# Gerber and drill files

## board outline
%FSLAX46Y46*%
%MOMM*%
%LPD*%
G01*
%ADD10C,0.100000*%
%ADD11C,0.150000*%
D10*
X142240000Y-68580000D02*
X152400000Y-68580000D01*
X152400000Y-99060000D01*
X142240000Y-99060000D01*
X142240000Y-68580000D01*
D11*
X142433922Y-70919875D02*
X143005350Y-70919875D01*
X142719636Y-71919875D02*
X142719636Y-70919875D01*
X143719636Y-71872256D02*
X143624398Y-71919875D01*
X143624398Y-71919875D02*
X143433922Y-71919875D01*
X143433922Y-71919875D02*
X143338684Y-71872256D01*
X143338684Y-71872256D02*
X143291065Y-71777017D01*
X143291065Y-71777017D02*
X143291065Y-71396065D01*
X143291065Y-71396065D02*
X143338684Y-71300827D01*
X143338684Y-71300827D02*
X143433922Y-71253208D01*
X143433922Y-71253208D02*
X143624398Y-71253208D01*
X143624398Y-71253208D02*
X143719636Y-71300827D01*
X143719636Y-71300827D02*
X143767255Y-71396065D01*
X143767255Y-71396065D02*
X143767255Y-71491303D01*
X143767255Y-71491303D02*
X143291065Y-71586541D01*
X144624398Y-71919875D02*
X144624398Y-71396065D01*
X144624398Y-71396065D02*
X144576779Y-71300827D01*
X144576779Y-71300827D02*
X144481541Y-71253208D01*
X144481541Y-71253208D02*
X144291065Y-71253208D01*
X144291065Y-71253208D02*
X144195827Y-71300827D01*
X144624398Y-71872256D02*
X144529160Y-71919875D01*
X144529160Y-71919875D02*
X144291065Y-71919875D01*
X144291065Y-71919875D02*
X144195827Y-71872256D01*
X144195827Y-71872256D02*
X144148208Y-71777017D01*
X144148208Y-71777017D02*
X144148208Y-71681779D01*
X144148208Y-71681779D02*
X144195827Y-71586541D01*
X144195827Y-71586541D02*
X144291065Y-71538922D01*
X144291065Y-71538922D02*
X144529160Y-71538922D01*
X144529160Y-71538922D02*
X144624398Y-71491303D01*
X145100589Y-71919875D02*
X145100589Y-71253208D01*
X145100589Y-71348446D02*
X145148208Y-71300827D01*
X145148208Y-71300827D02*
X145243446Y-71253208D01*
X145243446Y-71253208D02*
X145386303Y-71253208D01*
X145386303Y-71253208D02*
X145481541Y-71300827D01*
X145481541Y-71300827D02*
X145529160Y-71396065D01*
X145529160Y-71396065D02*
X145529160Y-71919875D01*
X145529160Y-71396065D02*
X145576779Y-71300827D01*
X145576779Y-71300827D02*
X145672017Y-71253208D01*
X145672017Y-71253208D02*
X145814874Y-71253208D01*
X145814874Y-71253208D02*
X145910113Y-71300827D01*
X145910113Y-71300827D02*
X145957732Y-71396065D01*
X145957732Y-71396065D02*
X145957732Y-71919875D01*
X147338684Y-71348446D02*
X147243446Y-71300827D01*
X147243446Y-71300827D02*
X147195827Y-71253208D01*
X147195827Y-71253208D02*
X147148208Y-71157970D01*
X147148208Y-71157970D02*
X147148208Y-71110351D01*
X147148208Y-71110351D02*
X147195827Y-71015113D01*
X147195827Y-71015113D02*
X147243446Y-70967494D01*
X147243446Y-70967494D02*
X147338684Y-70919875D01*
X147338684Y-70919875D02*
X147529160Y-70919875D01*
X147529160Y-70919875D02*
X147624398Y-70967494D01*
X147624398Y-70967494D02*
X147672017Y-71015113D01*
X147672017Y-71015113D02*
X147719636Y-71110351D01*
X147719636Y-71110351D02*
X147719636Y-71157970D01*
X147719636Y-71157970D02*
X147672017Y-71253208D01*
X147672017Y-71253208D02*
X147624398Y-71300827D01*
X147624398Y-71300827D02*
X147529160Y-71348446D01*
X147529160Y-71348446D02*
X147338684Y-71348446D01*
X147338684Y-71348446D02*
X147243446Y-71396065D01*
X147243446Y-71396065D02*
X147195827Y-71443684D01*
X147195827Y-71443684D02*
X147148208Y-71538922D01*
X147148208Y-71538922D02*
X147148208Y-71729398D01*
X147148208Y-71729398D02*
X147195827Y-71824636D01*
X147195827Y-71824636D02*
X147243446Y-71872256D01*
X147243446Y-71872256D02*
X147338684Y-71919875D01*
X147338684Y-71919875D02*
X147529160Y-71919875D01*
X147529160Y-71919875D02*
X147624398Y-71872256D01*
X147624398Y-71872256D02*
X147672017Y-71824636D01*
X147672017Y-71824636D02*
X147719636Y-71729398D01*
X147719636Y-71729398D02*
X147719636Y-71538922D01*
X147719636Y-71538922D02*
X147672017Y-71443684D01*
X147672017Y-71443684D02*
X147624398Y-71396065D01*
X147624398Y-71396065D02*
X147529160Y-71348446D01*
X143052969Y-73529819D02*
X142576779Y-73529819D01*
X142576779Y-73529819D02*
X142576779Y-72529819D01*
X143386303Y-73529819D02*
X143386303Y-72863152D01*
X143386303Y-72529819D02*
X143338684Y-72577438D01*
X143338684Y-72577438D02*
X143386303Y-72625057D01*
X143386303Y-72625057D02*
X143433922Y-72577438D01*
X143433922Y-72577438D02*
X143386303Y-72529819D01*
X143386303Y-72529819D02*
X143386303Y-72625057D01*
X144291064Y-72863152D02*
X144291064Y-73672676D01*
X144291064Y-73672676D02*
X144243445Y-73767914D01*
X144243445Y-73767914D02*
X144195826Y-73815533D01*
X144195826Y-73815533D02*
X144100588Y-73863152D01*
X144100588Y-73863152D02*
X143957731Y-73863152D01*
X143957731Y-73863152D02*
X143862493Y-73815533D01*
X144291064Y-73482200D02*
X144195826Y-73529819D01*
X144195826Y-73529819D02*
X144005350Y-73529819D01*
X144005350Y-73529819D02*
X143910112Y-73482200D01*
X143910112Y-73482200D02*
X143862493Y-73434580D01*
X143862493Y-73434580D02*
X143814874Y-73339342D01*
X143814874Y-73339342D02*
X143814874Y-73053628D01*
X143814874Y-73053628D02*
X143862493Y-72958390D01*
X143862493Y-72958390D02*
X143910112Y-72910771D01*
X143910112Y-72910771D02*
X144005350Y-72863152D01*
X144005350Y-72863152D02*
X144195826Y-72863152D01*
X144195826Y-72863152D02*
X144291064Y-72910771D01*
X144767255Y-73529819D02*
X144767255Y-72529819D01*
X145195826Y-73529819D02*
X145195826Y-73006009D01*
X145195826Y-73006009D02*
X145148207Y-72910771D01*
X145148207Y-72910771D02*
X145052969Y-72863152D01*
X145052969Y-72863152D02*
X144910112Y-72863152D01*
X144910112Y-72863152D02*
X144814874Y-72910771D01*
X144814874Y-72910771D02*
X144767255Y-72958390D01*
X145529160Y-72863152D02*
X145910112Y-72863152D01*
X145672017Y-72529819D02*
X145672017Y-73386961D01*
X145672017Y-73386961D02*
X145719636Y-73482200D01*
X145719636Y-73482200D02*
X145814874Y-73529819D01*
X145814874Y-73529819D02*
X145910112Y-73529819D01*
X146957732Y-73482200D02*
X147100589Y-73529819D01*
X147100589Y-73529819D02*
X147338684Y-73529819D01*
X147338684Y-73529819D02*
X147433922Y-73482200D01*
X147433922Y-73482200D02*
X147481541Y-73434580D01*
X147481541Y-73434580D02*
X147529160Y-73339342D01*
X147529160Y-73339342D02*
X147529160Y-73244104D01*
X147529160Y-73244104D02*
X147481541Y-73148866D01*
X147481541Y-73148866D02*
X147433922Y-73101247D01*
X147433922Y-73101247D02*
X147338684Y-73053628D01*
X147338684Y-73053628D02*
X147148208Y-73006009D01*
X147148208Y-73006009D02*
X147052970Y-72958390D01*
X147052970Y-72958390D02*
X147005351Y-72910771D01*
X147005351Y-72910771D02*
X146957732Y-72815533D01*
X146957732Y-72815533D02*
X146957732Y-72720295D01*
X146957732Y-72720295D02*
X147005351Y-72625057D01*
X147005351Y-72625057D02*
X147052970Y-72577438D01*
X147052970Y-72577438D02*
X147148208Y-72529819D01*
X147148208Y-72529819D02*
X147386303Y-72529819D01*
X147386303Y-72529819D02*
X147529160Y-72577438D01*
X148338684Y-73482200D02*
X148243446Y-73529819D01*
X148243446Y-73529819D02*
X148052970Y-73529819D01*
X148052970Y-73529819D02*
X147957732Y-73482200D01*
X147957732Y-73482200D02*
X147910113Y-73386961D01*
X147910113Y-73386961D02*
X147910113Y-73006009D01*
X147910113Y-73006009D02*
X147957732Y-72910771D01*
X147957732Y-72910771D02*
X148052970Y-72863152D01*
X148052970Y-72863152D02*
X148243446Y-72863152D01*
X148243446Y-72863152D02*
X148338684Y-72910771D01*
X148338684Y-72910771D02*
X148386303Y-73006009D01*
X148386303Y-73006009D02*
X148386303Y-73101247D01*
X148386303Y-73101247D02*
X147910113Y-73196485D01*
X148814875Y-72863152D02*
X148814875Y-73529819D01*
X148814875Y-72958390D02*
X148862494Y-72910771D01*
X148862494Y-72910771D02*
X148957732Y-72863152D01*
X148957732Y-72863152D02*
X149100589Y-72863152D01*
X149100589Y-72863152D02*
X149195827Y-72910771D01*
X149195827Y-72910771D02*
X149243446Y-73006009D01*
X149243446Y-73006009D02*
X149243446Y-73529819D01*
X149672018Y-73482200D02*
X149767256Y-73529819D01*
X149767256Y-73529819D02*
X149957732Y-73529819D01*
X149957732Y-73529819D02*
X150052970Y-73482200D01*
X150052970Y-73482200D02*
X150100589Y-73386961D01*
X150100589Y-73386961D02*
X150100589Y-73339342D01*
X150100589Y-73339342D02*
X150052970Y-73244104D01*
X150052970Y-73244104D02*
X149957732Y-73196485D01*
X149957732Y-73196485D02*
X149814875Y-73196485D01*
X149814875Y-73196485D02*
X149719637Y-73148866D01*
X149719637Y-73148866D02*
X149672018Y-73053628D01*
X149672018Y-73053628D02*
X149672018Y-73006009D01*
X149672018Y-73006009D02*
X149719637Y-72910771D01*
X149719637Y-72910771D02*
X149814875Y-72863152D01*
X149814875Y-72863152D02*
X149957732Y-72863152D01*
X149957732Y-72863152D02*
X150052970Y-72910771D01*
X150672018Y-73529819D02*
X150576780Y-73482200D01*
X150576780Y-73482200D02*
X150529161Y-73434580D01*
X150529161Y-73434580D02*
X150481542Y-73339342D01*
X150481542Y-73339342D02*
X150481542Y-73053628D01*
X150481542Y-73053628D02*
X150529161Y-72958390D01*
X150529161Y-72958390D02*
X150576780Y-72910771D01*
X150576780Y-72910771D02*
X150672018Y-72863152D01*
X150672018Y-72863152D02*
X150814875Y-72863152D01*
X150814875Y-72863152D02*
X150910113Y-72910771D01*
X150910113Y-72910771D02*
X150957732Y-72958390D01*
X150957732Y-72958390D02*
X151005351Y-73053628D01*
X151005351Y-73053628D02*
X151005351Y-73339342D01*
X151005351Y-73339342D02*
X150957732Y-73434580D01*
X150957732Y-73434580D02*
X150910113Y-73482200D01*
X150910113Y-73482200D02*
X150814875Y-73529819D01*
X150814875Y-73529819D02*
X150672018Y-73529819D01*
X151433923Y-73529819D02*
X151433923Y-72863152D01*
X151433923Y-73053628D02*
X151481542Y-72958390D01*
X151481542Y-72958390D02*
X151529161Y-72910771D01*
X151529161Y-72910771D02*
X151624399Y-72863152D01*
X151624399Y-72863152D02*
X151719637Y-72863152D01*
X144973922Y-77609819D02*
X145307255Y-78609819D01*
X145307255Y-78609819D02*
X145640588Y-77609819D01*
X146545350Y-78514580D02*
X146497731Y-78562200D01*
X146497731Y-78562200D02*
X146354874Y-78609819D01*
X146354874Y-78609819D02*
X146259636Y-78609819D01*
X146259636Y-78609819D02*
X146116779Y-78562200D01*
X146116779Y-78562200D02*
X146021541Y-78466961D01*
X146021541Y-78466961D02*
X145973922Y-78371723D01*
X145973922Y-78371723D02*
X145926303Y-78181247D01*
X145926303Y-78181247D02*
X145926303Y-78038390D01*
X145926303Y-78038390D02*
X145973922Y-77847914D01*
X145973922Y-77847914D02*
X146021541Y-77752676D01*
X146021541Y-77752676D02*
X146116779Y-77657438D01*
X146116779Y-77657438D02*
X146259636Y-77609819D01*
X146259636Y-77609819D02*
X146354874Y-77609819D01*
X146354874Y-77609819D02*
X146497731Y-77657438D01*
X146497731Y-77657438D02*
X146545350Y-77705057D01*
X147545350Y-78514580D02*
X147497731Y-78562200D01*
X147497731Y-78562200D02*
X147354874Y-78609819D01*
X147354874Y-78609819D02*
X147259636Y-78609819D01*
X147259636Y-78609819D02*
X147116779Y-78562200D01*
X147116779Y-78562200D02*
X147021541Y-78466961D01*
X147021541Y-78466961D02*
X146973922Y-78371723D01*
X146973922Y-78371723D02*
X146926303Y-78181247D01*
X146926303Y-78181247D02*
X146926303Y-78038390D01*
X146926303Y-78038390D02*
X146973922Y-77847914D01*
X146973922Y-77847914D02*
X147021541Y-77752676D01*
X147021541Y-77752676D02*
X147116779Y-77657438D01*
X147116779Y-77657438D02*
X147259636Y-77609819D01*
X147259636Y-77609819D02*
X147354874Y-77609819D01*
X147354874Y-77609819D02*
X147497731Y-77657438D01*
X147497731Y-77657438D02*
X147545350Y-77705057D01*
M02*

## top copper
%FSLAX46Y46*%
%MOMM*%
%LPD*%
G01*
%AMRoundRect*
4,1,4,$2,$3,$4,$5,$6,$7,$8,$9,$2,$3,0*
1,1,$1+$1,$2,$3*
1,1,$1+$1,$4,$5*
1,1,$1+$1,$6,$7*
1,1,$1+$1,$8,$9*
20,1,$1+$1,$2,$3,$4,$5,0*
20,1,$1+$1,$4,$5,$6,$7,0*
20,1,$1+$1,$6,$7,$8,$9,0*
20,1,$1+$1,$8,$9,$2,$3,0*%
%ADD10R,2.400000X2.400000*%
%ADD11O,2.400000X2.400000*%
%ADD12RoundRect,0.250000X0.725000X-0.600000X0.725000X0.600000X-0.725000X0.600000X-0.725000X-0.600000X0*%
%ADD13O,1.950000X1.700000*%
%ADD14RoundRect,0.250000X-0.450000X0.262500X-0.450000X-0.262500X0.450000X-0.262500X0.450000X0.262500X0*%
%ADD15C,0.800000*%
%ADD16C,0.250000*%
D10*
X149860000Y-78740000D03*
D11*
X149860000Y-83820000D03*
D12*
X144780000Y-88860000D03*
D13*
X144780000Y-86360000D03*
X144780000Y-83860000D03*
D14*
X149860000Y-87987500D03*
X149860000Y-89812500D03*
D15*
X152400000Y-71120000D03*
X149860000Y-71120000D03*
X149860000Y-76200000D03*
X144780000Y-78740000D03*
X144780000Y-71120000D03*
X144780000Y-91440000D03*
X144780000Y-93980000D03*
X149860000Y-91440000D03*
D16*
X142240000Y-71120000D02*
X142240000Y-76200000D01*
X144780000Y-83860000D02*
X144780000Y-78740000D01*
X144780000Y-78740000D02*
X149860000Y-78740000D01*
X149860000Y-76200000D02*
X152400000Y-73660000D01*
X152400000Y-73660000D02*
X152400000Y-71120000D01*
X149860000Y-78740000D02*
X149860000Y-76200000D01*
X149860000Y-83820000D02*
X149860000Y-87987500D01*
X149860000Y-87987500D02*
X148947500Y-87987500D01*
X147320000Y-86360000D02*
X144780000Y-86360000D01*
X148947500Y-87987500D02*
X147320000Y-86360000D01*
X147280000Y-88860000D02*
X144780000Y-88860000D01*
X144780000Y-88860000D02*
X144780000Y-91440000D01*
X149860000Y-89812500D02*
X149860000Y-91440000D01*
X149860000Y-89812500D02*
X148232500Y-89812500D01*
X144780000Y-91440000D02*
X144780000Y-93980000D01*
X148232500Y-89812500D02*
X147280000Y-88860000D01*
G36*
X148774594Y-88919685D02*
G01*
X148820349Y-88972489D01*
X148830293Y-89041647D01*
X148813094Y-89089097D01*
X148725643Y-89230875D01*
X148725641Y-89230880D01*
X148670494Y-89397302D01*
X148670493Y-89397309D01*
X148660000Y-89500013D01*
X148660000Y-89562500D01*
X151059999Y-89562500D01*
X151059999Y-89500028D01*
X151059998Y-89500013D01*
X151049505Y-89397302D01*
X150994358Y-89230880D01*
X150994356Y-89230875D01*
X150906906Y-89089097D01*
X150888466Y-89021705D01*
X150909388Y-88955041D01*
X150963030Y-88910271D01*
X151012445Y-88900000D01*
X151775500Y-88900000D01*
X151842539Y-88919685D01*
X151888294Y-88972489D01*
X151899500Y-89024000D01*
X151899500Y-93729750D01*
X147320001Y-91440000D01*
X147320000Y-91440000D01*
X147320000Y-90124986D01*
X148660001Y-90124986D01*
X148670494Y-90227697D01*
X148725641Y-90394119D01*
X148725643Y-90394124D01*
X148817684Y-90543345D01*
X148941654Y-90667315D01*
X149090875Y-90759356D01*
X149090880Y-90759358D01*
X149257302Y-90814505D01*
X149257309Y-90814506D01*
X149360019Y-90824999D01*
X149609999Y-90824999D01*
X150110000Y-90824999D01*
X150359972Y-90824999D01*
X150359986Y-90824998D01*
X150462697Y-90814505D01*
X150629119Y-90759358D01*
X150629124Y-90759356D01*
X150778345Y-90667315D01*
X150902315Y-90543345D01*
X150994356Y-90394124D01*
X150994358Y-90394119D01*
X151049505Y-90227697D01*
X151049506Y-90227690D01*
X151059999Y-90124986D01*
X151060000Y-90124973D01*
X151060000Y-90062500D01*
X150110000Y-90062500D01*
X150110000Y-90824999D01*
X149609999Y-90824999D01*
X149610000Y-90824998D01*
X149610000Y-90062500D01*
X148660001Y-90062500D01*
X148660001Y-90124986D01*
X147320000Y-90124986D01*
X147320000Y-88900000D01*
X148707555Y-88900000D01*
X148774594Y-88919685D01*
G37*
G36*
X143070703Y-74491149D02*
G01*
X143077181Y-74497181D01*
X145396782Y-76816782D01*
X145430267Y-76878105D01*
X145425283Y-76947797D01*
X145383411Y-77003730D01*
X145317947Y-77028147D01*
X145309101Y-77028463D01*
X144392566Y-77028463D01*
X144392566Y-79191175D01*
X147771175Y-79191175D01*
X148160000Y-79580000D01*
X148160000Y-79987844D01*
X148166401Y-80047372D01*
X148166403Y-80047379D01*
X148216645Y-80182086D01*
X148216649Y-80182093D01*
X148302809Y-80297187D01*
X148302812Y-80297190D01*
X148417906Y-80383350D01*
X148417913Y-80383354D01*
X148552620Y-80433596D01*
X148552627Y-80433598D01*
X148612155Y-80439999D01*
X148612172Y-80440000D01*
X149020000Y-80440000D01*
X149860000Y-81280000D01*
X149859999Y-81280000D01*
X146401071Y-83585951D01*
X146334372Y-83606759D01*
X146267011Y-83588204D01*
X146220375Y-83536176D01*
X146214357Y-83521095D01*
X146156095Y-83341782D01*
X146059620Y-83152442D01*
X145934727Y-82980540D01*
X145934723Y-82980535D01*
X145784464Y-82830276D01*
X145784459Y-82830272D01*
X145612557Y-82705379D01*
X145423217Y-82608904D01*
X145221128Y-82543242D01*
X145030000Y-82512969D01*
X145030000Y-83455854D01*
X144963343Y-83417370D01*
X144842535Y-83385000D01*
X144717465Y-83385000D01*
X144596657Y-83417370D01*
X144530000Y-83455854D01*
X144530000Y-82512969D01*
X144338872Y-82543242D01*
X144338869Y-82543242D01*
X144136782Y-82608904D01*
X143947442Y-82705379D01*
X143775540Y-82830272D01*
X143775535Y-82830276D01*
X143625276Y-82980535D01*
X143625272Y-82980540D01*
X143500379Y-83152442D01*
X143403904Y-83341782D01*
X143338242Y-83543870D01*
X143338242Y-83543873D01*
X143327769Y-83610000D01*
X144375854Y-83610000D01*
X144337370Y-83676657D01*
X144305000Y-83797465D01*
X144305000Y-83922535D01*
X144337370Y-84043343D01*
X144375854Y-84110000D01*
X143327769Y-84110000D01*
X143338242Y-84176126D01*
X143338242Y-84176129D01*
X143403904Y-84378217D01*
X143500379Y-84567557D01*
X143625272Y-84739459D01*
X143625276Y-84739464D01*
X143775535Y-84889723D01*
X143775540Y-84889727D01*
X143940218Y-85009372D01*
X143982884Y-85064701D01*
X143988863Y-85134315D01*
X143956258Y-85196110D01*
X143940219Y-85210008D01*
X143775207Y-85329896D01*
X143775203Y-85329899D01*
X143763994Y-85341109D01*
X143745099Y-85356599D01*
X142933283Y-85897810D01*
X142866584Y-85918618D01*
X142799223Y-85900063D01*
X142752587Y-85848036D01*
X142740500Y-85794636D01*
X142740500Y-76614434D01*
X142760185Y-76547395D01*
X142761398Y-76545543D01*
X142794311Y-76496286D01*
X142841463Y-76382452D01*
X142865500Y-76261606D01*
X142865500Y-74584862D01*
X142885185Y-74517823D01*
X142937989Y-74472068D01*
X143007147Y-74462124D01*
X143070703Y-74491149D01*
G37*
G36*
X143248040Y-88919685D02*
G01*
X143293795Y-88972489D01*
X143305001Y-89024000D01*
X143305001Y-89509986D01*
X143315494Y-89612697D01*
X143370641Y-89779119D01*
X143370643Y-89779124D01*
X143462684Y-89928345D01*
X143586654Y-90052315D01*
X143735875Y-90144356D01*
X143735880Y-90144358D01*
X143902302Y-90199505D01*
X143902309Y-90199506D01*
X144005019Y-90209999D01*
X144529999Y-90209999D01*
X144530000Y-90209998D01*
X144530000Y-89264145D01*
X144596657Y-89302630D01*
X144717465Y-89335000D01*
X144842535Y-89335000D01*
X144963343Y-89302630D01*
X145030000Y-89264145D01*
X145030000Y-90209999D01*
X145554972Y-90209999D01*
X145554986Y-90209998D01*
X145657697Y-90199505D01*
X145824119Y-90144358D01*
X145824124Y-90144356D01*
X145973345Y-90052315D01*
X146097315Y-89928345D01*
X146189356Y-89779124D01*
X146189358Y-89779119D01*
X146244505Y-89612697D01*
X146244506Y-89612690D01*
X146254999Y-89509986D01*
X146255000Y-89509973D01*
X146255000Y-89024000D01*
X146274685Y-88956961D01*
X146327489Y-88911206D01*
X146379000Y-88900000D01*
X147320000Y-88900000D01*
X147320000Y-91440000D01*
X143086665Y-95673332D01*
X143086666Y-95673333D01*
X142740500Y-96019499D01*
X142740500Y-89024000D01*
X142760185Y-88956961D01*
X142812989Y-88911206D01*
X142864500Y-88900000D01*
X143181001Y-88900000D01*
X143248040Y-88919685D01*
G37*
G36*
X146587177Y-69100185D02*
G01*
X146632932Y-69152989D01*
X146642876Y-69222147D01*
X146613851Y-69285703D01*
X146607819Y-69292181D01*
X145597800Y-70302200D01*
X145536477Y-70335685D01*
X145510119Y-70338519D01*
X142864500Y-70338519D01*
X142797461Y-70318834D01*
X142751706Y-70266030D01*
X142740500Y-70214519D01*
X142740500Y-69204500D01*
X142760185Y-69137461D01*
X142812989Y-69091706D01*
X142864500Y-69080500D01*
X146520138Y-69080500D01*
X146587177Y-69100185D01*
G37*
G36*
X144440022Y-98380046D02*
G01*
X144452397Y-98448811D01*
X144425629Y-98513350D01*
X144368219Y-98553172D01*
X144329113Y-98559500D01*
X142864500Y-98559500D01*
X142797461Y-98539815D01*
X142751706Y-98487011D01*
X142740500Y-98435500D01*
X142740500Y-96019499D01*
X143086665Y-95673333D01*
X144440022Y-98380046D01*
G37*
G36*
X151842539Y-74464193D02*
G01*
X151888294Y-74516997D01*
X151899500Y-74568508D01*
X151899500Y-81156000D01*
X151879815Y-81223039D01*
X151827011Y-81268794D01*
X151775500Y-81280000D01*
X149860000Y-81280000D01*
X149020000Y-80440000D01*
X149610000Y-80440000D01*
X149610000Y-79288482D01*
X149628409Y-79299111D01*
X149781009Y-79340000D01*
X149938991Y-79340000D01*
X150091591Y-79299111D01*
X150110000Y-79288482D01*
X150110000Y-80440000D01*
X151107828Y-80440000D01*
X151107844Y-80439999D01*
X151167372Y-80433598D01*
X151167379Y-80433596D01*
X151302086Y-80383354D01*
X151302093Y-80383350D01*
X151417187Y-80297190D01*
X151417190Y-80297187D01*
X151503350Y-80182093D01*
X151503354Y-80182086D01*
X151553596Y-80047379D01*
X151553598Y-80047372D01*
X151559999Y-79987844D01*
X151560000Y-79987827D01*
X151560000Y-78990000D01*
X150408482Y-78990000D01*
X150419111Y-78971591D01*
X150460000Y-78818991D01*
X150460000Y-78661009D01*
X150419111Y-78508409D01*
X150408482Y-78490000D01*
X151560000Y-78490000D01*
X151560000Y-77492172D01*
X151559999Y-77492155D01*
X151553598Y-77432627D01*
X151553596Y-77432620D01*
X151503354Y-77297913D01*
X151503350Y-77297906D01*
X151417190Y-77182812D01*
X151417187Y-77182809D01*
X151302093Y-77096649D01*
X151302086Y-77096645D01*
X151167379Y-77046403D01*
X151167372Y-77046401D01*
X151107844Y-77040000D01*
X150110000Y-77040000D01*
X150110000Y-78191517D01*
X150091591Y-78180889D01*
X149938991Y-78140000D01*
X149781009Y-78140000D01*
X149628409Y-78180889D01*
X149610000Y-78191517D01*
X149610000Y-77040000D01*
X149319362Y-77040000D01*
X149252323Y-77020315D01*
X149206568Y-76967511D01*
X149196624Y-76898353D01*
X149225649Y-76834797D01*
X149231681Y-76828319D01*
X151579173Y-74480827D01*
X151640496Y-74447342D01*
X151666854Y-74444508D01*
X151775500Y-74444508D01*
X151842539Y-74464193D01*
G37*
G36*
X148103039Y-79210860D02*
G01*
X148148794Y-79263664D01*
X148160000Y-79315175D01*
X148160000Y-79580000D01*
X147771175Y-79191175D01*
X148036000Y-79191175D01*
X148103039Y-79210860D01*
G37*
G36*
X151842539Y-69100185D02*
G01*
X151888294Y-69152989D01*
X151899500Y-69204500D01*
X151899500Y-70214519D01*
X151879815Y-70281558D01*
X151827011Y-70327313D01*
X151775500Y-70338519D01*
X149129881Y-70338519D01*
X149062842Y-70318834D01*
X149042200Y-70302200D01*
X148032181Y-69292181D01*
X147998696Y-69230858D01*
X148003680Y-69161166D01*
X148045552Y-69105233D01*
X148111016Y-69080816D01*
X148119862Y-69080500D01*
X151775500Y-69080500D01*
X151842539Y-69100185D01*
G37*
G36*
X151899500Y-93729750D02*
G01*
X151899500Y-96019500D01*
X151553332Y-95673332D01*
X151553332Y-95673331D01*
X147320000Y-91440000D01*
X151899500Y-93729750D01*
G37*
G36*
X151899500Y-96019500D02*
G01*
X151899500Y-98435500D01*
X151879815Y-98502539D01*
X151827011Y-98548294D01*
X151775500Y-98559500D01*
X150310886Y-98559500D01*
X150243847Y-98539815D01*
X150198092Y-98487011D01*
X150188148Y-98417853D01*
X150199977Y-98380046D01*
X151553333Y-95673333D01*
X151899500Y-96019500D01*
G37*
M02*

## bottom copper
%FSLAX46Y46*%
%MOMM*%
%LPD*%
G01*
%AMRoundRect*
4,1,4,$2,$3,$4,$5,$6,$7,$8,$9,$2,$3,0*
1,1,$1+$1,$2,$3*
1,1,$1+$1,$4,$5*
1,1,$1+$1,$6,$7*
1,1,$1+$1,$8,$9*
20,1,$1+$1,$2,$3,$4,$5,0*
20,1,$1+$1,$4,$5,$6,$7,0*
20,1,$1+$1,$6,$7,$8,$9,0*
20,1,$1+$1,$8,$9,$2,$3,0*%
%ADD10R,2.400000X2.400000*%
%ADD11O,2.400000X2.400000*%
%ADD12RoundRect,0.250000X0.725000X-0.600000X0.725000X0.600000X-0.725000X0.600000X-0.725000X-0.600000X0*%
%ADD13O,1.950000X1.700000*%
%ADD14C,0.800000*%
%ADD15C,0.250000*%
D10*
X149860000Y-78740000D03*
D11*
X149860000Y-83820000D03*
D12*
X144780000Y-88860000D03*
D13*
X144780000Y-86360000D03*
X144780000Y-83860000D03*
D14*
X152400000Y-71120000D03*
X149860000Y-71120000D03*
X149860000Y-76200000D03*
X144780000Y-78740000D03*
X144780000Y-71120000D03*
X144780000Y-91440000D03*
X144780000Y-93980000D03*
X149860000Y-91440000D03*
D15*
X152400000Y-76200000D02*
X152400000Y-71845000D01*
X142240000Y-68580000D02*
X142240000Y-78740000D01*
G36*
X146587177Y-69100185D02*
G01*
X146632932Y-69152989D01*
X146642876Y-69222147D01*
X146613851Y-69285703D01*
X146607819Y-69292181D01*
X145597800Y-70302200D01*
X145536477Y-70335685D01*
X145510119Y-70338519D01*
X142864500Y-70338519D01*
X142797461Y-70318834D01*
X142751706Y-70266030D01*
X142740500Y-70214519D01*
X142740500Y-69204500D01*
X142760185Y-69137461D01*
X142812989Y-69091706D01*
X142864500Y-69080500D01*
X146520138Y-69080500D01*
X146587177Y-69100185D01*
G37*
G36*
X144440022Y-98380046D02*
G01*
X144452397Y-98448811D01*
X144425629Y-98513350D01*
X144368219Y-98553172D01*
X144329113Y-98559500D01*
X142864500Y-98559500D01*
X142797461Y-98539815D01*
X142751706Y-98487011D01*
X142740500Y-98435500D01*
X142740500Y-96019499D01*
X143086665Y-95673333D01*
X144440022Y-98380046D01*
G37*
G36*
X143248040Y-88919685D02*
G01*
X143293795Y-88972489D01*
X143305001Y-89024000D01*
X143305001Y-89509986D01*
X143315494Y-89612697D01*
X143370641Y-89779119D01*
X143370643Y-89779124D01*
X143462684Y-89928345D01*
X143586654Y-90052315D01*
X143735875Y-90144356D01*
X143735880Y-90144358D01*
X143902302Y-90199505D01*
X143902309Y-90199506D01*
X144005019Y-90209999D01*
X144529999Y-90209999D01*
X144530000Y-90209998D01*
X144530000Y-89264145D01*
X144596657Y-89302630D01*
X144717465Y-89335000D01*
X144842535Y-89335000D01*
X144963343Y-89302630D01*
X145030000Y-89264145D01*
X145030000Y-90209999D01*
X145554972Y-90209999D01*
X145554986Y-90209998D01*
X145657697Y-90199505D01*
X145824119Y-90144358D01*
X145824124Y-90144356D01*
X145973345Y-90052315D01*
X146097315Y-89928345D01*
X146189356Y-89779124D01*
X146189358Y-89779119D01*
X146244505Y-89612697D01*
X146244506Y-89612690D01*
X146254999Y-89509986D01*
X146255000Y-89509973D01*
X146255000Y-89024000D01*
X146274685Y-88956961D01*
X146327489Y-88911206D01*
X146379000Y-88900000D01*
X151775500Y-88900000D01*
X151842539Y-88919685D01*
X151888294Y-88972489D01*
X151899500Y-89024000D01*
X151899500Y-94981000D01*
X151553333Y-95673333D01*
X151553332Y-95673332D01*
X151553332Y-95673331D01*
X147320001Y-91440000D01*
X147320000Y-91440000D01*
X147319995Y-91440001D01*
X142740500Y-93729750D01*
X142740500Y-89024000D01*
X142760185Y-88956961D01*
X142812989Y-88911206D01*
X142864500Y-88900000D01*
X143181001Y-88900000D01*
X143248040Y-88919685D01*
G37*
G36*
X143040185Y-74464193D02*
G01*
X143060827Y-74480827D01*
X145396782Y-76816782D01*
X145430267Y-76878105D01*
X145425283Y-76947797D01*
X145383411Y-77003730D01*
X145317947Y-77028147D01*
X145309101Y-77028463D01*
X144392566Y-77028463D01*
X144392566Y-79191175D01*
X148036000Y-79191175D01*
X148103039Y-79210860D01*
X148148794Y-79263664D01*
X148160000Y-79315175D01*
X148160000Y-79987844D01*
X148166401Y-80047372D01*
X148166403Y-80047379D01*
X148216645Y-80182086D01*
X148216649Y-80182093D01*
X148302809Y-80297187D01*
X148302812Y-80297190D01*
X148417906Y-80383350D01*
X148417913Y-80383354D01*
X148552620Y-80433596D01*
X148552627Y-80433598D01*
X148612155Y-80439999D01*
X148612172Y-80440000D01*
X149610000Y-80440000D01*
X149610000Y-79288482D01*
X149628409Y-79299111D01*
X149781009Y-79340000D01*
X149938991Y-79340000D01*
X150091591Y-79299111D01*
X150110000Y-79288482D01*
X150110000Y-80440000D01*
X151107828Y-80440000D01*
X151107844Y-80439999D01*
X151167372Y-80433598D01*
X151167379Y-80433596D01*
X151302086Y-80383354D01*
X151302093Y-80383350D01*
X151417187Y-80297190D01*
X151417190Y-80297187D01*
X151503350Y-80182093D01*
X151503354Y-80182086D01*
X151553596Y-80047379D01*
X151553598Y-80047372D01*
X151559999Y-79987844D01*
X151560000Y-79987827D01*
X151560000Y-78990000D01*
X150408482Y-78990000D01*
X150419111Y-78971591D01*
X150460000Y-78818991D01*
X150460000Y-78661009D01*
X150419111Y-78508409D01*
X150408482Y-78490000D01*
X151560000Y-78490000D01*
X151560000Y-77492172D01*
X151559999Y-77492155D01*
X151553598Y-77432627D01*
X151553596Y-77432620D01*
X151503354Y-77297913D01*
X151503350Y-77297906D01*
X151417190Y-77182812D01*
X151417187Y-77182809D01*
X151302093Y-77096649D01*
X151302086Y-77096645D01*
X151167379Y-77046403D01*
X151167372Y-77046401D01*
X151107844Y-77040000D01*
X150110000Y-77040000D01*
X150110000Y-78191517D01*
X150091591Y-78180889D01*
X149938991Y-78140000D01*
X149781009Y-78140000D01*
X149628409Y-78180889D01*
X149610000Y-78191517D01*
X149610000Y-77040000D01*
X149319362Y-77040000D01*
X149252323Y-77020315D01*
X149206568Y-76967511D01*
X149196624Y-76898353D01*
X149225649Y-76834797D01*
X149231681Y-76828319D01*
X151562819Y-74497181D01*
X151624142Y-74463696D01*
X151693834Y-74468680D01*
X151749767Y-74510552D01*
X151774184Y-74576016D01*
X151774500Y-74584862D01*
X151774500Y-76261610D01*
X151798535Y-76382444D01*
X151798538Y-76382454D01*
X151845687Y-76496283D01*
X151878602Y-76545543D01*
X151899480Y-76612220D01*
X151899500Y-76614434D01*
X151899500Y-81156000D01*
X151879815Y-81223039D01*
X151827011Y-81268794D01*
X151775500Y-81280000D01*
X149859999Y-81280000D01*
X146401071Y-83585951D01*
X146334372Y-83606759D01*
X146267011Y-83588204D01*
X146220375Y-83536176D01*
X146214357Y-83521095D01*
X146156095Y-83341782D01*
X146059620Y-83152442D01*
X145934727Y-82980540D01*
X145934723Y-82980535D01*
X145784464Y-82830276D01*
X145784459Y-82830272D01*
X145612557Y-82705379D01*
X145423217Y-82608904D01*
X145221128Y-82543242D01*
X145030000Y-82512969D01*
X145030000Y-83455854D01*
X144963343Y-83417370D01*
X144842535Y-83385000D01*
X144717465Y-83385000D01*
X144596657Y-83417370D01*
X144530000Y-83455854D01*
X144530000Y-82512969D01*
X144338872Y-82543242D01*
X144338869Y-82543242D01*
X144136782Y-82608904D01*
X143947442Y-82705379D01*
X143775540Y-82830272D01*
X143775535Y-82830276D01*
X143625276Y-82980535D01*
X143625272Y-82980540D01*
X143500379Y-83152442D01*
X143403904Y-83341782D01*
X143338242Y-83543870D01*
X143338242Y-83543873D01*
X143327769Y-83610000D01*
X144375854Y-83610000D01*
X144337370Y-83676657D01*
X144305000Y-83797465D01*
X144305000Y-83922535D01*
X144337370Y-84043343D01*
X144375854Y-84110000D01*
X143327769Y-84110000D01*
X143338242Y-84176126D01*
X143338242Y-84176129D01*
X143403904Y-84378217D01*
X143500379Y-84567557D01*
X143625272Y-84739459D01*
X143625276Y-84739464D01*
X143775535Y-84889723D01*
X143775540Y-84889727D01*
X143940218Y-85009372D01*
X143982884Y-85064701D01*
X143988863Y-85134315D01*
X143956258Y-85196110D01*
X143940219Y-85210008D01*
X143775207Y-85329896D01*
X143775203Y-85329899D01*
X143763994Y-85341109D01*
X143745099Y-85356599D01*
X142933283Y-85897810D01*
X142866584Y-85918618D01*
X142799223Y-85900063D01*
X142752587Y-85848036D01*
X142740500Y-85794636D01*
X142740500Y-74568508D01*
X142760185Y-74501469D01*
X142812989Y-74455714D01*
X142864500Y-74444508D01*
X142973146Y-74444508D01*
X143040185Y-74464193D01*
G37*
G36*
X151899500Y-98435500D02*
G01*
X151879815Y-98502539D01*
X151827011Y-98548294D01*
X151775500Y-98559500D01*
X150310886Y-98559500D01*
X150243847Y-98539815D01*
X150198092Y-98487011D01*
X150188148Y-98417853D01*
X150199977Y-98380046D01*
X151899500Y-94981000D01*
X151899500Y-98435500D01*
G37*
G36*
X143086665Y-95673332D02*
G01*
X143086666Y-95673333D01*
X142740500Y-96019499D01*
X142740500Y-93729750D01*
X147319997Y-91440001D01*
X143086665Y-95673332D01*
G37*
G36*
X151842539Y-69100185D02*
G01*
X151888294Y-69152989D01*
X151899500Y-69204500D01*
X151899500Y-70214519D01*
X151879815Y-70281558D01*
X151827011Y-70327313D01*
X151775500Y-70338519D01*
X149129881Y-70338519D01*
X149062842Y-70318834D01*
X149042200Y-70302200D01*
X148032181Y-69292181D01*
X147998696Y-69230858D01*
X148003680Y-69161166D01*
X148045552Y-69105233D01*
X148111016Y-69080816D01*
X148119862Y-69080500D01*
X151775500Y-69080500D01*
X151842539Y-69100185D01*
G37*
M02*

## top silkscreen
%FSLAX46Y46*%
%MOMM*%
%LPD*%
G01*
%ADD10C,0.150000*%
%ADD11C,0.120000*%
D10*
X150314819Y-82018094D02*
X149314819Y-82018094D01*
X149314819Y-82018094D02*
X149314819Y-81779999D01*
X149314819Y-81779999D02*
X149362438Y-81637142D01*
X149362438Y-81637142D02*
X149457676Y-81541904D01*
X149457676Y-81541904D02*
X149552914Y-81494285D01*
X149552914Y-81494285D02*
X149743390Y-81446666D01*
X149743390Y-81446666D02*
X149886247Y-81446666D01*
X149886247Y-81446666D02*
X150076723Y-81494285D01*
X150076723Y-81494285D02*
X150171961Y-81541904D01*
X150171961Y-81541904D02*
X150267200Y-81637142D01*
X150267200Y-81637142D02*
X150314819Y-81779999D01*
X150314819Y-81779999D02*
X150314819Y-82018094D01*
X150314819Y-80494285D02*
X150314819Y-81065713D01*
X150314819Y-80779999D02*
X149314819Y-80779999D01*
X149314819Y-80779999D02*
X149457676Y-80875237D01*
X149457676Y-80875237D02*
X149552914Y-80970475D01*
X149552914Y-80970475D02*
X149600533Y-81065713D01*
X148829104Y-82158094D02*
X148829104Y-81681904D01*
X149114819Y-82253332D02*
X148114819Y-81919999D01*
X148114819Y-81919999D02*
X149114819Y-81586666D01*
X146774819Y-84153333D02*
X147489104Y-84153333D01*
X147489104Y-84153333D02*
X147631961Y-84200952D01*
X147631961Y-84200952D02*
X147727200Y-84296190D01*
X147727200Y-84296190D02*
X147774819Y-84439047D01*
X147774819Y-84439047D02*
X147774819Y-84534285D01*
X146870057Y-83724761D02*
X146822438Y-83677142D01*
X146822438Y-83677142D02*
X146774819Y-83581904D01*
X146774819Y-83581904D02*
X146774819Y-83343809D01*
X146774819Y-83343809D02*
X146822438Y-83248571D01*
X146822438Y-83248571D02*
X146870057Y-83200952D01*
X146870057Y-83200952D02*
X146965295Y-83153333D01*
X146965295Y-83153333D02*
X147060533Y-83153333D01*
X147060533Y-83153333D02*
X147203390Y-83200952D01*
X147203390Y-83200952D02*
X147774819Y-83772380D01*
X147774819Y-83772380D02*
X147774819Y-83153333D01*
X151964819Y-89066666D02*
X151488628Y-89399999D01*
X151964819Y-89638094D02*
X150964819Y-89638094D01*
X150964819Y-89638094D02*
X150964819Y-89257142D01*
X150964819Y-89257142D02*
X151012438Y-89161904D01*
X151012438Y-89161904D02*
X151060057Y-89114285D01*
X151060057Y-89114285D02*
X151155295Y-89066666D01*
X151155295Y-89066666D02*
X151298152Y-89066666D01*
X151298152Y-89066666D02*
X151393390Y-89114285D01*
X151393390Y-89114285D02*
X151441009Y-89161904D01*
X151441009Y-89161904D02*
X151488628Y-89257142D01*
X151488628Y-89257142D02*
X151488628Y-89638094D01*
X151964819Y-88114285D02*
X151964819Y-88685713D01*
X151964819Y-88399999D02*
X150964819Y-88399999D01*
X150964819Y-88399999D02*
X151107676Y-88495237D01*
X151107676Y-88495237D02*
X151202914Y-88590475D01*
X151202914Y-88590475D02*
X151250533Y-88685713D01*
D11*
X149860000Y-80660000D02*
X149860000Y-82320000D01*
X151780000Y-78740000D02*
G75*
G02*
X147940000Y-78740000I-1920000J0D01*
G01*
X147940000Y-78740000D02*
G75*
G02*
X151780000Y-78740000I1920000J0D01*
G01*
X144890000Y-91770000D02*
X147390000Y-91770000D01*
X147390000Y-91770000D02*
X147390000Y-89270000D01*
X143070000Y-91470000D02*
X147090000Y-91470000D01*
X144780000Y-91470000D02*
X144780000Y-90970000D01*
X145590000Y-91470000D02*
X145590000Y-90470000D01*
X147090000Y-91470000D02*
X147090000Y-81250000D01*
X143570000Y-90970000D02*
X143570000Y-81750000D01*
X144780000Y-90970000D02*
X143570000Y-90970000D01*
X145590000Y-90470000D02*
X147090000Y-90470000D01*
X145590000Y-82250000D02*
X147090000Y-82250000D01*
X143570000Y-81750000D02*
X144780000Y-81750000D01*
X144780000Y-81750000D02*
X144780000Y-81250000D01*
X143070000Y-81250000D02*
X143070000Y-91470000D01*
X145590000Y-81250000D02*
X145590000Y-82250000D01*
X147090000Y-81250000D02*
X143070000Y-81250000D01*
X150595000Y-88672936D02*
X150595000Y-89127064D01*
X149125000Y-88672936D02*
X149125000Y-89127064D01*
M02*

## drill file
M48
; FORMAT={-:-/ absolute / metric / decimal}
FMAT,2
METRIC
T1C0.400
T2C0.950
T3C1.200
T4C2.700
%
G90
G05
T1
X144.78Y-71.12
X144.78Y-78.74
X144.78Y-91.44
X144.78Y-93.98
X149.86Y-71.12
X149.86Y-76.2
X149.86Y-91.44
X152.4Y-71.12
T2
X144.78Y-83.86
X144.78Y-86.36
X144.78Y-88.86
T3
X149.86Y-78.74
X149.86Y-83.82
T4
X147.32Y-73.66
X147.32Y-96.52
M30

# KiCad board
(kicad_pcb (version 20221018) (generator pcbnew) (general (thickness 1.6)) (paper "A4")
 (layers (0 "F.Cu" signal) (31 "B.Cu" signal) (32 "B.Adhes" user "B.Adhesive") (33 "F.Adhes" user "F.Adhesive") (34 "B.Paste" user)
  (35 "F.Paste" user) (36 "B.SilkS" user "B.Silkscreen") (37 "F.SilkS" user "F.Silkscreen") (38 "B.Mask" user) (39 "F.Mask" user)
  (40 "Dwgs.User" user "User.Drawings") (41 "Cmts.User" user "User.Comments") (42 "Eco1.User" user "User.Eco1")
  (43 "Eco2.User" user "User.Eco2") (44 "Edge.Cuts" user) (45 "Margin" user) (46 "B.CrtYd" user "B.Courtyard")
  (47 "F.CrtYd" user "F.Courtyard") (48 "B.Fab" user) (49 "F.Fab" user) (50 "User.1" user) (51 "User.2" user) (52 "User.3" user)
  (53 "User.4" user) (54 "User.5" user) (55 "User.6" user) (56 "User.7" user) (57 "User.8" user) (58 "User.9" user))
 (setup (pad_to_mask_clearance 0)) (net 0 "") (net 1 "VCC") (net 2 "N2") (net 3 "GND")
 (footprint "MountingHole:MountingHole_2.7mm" (layer "F.Cu") (at 147.32 96.52)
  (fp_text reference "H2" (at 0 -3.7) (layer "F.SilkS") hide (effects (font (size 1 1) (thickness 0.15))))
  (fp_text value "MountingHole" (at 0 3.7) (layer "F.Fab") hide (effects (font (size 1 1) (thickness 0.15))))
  (pad "" np_thru_hole circle (at 0 0) (size 2.7 2.7) (drill 2.7) (layers "*.Cu" "*.Mask")))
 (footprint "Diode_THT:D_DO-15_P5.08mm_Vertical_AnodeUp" (layer "F.Cu") (at 149.86 78.74 -90)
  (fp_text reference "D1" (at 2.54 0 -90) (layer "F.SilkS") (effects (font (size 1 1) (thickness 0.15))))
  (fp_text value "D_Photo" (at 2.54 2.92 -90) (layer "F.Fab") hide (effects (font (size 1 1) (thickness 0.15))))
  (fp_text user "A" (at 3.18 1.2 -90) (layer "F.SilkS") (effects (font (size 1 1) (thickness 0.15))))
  (fp_line (start 1.92 0) (end 3.58 0) (stroke (width 0.12) (type solid)) (layer "F.SilkS"))
  (fp_circle (center 0 0) (end 1.92 0) (stroke (width 0.12) (type solid)) (fill none) (layer "F.SilkS"))
  (pad "1" thru_hole rect (at 0 0 270) (size 2.4 2.4) (drill 1.2) (layers "*.Cu" "*.Mask") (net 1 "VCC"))
  (pad "2" thru_hole oval (at 5.08 0 270) (size 2.4 2.4) (drill 1.2) (layers "*.Cu" "*.Mask") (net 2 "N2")))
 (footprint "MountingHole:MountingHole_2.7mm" (layer "F.Cu") (at 147.32 73.66)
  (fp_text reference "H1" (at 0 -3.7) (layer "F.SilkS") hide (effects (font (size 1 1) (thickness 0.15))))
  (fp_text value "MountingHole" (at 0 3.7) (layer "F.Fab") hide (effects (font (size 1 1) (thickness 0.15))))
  (pad "" np_thru_hole circle (at 0 0) (size 2.7 2.7) (drill 2.7) (layers "*.Cu" "*.Mask")))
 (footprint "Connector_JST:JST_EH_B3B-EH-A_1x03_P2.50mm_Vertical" (layer "F.Cu") (at 144.78 88.86 90)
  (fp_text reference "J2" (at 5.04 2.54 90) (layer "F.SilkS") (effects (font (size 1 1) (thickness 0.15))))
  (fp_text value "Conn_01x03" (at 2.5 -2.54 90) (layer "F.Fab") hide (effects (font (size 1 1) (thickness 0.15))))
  (fp_line (start -2.91 0.11) (end -2.91 2.61) (stroke (width 0.12) (type solid)) (layer "F.SilkS"))
  (fp_line (start -2.91 2.61) (end -0.41 2.61) (stroke (width 0.12) (type solid)) (layer "F.SilkS"))
  (fp_line (start -2.61 -1.71) (end -2.61 2.31) (stroke (width 0.12) (type solid)) (layer "F.SilkS"))
  (fp_line (start -2.61 0) (end -2.11 0) (stroke (width 0.12) (type solid)) (layer "F.SilkS"))
  (fp_line (start -2.61 0.81) (end -1.61 0.81) (stroke (width 0.12) (type solid)) (layer "F.SilkS"))
  (fp_line (start -2.61 2.31) (end 7.61 2.31) (stroke (width 0.12) (type solid)) (layer "F.SilkS"))
  (fp_line (start -2.11 -1.21) (end 7.11 -1.21) (stroke (width 0.12) (type solid)) (layer "F.SilkS"))
  (fp_line (start -2.11 0) (end -2.11 -1.21) (stroke (width 0.12) (type solid)) (layer "F.SilkS"))
  (fp_line (start -1.61 0.81) (end -1.61 2.31) (stroke (width 0.12) (type solid)) (layer "F.SilkS"))
  (fp_line (start 6.61 0.81) (end 6.61 2.31) (stroke (width 0.12) (type solid)) (layer "F.SilkS"))
  (fp_line (start 7.11 -1.21) (end 7.11 0) (stroke (width 0.12) (type solid)) (layer "F.SilkS"))
  (fp_line (start 7.11 0) (end 7.61 0) (stroke (width 0.12) (type solid)) (layer "F.SilkS"))
  (fp_line (start 7.61 -1.71) (end -2.61 -1.71) (stroke (width 0.12) (type solid)) (layer "F.SilkS"))
  (fp_line (start 7.61 0.81) (end 6.61 0.81) (stroke (width 0.12) (type solid)) (layer "F.SilkS"))
  (fp_line (start 7.61 2.31) (end 7.61 -1.71) (stroke (width 0.12) (type solid)) (layer "F.SilkS"))
  (pad "1" thru_hole roundrect (at 0 0 90) (size 1.7 1.95) (drill 0.95) (layers "*.Cu" "*.Mask") (roundrect_rratio 0.1470588235)
   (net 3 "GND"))
  (pad "2" thru_hole oval (at 2.5 0 90) (size 1.7 1.95) (drill 0.95) (layers "*.Cu" "*.Mask") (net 2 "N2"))
  (pad "3" thru_hole oval (at 5 0 90) (size 1.7 1.95) (drill 0.95) (layers "*.Cu" "*.Mask") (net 1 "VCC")))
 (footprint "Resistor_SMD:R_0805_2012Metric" (layer "F.Cu") (at 149.86 88.9 -90)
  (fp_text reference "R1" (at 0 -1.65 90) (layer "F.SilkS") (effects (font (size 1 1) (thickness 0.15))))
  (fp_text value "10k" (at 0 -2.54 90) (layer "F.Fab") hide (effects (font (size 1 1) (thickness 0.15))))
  (fp_line (start -0.227064 -0.735) (end 0.227064 -0.735) (stroke (width 0.12) (type solid)) (layer "F.SilkS"))
  (fp_line (start -0.227064 0.735) (end 0.227064 0.735) (stroke (width 0.12) (type solid)) (layer "F.SilkS"))
  (pad "1" smd roundrect (at -0.9125 0 270) (size 1.025 1.4) (layers "F.Cu" "F.Paste" "F.Mask") (roundrect_rratio 0.243902439) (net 2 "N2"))
  (pad "2" smd roundrect (at 0.9125 0 270) (size 1.025 1.4) (layers "F.Cu" "F.Paste" "F.Mask") (roundrect_rratio 0.243902439) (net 3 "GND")))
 (gr_rect (start 142.24 68.58) (end 152.4 99.06) (stroke (width 0.1) (type default)) (fill none) (layer "Edge.Cuts"))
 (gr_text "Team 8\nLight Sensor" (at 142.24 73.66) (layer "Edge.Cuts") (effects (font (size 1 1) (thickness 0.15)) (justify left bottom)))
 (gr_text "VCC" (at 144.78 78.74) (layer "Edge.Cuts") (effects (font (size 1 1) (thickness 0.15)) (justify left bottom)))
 (segment (start 142.24 71.12) (end 142.24 76.2) (width 0.25) (layer "F.Cu") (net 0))
 (segment (start 152.4 76.2) (end 152.4 71.845) (width 0.25) (layer "B.Cu") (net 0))
 (segment (start 144.78 83.86) (end 144.78 78.74) (width 0.25) (layer "F.Cu") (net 1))
 (segment (start 144.78 78.74) (end 149.86 78.74) (width 0.25) (layer "F.Cu") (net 1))
 (segment (start 149.86 76.2) (end 152.4 73.66) (width 0.25) (layer "F.Cu") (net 1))
 (segment (start 152.4 73.66) (end 152.4 71.12) (width 0.25) (layer "F.Cu") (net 1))
 (segment (start 149.86 78.74) (end 149.86 76.2) (width 0.25) (layer "F.Cu") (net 1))
 (via (at 152.4 71.12) (size 0.8) (drill 0.4) (layers "F.Cu" "B.Cu") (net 1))
 (via (at 149.86 71.12) (size 0.8) (drill 0.4) (layers "F.Cu" "B.Cu") (free) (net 1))
 (via (at 149.86 76.2) (size 0.8) (drill 0.4) (layers "F.Cu" "B.Cu") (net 1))
 (via (at 144.78 78.74) (size 0.8) (drill 0.4) (layers "F.Cu" "B.Cu") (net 1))
 (via (at 144.78 71.12) (size 0.8) (drill 0.4) (layers "F.Cu" "B.Cu") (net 1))
 (segment (start 142.24 68.58) (end 142.24 78.74) (width 0.25) (layer "B.Cu") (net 1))
 (segment (start 149.86 83.82) (end 149.86 87.9875) (width 0.25) (layer "F.Cu") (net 2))
 (segment (start 149.86 87.9875) (end 148.9475 87.9875) (width 0.25) (layer "F.Cu") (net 2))
 (segment (start 147.32 86.36) (end 144.78 86.36) (width 0.25) (layer "F.Cu") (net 2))
 (segment (start 148.9475 87.9875) (end 147.32 86.36) (width 0.25) (layer "F.Cu") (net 2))
 (segment (start 147.28 88.86) (end 144.78 88.86) (width 0.25) (layer "F.Cu") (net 3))
 (segment (start 144.78 88.86) (end 144.78 91.44) (width 0.25) (layer "F.Cu") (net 3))
 (segment (start 149.86 89.8125) (end 149.86 91.44) (width 0.25) (layer "F.Cu") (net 3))
 (segment (start 149.86 89.8125) (end 148.2325 89.8125) (width 0.25) (layer "F.Cu") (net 3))
 (segment (start 144.78 91.44) (end 144.78 93.98) (width 0.25) (layer "F.Cu") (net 3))
 (segment (start 148.2325 89.8125) (end 147.28 88.86) (width 0.25) (layer "F.Cu") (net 3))
 (via (at 144.78 91.44) (size 0.8) (drill 0.4) (layers "F.Cu" "B.Cu") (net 3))
 (via (at 144.78 93.98) (size 0.8) (drill 0.4) (layers "F.Cu" "B.Cu") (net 3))
 (via (at 149.86 91.44) (size 0.8) (drill 0.4) (layers "F.Cu" "B.Cu") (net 3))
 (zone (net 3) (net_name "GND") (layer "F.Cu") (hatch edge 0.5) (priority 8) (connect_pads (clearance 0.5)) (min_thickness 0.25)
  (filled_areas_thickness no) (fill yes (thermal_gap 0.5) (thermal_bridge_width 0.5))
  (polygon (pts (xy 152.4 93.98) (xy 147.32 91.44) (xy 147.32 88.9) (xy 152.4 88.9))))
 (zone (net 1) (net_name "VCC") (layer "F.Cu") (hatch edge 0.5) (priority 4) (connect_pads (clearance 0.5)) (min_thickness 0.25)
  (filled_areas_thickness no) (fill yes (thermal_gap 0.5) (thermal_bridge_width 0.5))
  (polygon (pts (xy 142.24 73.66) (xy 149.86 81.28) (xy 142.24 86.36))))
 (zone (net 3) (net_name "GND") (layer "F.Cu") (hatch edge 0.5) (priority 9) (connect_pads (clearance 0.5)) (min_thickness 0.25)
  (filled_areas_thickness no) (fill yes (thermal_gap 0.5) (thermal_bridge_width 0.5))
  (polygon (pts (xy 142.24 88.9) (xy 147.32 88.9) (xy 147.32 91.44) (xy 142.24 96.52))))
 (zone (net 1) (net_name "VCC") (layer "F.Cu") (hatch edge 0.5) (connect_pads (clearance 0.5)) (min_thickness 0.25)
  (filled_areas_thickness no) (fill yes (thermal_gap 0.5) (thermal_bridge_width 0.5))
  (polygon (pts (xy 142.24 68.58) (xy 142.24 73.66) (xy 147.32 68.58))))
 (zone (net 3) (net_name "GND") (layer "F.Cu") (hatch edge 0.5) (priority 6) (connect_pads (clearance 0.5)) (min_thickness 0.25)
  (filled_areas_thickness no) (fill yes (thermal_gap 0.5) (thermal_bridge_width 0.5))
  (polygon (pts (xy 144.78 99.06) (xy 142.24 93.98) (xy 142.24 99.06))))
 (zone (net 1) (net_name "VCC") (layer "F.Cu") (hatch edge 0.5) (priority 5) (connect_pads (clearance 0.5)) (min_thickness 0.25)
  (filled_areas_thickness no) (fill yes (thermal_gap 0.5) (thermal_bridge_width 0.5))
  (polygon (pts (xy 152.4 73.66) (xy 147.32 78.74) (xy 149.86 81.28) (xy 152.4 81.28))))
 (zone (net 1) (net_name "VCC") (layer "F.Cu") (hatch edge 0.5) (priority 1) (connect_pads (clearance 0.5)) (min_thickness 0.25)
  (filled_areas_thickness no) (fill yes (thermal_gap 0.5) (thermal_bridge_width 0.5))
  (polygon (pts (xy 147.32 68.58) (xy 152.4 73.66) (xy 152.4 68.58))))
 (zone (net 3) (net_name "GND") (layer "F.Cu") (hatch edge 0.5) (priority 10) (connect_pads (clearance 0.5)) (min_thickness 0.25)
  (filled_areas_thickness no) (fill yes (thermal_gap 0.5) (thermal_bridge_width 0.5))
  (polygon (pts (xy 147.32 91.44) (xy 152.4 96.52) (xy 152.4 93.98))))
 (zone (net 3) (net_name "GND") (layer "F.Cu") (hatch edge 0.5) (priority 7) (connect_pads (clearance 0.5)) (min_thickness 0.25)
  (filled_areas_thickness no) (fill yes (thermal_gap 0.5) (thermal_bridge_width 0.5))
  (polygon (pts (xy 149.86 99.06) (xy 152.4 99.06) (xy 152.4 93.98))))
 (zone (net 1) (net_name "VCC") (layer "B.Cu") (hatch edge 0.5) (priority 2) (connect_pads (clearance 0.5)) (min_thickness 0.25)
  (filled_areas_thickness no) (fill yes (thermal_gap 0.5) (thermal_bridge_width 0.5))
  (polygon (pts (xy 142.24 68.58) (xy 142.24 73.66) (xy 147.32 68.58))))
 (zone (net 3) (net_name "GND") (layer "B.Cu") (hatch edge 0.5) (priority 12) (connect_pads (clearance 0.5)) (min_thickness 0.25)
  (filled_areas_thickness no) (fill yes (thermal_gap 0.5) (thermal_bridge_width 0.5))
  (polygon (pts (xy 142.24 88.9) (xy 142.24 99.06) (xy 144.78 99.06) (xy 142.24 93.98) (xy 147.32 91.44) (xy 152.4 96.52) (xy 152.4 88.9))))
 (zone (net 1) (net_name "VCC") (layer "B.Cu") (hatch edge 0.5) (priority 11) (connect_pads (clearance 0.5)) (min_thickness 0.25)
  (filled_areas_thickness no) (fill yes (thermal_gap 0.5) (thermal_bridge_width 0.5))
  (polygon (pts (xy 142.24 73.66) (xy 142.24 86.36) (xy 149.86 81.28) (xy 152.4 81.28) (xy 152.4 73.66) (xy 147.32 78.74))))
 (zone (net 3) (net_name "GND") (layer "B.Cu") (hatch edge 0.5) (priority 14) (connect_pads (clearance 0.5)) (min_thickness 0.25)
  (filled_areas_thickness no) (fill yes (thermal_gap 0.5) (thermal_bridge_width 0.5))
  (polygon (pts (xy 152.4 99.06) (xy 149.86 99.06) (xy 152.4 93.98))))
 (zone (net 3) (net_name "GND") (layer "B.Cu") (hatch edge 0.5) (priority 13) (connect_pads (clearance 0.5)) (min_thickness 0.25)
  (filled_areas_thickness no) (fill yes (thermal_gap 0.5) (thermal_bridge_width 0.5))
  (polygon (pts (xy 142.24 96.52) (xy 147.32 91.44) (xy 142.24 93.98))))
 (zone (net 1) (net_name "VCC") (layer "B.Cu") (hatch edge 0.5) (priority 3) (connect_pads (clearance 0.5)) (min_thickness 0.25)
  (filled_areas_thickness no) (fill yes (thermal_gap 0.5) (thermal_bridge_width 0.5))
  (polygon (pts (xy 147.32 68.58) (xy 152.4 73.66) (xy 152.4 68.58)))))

